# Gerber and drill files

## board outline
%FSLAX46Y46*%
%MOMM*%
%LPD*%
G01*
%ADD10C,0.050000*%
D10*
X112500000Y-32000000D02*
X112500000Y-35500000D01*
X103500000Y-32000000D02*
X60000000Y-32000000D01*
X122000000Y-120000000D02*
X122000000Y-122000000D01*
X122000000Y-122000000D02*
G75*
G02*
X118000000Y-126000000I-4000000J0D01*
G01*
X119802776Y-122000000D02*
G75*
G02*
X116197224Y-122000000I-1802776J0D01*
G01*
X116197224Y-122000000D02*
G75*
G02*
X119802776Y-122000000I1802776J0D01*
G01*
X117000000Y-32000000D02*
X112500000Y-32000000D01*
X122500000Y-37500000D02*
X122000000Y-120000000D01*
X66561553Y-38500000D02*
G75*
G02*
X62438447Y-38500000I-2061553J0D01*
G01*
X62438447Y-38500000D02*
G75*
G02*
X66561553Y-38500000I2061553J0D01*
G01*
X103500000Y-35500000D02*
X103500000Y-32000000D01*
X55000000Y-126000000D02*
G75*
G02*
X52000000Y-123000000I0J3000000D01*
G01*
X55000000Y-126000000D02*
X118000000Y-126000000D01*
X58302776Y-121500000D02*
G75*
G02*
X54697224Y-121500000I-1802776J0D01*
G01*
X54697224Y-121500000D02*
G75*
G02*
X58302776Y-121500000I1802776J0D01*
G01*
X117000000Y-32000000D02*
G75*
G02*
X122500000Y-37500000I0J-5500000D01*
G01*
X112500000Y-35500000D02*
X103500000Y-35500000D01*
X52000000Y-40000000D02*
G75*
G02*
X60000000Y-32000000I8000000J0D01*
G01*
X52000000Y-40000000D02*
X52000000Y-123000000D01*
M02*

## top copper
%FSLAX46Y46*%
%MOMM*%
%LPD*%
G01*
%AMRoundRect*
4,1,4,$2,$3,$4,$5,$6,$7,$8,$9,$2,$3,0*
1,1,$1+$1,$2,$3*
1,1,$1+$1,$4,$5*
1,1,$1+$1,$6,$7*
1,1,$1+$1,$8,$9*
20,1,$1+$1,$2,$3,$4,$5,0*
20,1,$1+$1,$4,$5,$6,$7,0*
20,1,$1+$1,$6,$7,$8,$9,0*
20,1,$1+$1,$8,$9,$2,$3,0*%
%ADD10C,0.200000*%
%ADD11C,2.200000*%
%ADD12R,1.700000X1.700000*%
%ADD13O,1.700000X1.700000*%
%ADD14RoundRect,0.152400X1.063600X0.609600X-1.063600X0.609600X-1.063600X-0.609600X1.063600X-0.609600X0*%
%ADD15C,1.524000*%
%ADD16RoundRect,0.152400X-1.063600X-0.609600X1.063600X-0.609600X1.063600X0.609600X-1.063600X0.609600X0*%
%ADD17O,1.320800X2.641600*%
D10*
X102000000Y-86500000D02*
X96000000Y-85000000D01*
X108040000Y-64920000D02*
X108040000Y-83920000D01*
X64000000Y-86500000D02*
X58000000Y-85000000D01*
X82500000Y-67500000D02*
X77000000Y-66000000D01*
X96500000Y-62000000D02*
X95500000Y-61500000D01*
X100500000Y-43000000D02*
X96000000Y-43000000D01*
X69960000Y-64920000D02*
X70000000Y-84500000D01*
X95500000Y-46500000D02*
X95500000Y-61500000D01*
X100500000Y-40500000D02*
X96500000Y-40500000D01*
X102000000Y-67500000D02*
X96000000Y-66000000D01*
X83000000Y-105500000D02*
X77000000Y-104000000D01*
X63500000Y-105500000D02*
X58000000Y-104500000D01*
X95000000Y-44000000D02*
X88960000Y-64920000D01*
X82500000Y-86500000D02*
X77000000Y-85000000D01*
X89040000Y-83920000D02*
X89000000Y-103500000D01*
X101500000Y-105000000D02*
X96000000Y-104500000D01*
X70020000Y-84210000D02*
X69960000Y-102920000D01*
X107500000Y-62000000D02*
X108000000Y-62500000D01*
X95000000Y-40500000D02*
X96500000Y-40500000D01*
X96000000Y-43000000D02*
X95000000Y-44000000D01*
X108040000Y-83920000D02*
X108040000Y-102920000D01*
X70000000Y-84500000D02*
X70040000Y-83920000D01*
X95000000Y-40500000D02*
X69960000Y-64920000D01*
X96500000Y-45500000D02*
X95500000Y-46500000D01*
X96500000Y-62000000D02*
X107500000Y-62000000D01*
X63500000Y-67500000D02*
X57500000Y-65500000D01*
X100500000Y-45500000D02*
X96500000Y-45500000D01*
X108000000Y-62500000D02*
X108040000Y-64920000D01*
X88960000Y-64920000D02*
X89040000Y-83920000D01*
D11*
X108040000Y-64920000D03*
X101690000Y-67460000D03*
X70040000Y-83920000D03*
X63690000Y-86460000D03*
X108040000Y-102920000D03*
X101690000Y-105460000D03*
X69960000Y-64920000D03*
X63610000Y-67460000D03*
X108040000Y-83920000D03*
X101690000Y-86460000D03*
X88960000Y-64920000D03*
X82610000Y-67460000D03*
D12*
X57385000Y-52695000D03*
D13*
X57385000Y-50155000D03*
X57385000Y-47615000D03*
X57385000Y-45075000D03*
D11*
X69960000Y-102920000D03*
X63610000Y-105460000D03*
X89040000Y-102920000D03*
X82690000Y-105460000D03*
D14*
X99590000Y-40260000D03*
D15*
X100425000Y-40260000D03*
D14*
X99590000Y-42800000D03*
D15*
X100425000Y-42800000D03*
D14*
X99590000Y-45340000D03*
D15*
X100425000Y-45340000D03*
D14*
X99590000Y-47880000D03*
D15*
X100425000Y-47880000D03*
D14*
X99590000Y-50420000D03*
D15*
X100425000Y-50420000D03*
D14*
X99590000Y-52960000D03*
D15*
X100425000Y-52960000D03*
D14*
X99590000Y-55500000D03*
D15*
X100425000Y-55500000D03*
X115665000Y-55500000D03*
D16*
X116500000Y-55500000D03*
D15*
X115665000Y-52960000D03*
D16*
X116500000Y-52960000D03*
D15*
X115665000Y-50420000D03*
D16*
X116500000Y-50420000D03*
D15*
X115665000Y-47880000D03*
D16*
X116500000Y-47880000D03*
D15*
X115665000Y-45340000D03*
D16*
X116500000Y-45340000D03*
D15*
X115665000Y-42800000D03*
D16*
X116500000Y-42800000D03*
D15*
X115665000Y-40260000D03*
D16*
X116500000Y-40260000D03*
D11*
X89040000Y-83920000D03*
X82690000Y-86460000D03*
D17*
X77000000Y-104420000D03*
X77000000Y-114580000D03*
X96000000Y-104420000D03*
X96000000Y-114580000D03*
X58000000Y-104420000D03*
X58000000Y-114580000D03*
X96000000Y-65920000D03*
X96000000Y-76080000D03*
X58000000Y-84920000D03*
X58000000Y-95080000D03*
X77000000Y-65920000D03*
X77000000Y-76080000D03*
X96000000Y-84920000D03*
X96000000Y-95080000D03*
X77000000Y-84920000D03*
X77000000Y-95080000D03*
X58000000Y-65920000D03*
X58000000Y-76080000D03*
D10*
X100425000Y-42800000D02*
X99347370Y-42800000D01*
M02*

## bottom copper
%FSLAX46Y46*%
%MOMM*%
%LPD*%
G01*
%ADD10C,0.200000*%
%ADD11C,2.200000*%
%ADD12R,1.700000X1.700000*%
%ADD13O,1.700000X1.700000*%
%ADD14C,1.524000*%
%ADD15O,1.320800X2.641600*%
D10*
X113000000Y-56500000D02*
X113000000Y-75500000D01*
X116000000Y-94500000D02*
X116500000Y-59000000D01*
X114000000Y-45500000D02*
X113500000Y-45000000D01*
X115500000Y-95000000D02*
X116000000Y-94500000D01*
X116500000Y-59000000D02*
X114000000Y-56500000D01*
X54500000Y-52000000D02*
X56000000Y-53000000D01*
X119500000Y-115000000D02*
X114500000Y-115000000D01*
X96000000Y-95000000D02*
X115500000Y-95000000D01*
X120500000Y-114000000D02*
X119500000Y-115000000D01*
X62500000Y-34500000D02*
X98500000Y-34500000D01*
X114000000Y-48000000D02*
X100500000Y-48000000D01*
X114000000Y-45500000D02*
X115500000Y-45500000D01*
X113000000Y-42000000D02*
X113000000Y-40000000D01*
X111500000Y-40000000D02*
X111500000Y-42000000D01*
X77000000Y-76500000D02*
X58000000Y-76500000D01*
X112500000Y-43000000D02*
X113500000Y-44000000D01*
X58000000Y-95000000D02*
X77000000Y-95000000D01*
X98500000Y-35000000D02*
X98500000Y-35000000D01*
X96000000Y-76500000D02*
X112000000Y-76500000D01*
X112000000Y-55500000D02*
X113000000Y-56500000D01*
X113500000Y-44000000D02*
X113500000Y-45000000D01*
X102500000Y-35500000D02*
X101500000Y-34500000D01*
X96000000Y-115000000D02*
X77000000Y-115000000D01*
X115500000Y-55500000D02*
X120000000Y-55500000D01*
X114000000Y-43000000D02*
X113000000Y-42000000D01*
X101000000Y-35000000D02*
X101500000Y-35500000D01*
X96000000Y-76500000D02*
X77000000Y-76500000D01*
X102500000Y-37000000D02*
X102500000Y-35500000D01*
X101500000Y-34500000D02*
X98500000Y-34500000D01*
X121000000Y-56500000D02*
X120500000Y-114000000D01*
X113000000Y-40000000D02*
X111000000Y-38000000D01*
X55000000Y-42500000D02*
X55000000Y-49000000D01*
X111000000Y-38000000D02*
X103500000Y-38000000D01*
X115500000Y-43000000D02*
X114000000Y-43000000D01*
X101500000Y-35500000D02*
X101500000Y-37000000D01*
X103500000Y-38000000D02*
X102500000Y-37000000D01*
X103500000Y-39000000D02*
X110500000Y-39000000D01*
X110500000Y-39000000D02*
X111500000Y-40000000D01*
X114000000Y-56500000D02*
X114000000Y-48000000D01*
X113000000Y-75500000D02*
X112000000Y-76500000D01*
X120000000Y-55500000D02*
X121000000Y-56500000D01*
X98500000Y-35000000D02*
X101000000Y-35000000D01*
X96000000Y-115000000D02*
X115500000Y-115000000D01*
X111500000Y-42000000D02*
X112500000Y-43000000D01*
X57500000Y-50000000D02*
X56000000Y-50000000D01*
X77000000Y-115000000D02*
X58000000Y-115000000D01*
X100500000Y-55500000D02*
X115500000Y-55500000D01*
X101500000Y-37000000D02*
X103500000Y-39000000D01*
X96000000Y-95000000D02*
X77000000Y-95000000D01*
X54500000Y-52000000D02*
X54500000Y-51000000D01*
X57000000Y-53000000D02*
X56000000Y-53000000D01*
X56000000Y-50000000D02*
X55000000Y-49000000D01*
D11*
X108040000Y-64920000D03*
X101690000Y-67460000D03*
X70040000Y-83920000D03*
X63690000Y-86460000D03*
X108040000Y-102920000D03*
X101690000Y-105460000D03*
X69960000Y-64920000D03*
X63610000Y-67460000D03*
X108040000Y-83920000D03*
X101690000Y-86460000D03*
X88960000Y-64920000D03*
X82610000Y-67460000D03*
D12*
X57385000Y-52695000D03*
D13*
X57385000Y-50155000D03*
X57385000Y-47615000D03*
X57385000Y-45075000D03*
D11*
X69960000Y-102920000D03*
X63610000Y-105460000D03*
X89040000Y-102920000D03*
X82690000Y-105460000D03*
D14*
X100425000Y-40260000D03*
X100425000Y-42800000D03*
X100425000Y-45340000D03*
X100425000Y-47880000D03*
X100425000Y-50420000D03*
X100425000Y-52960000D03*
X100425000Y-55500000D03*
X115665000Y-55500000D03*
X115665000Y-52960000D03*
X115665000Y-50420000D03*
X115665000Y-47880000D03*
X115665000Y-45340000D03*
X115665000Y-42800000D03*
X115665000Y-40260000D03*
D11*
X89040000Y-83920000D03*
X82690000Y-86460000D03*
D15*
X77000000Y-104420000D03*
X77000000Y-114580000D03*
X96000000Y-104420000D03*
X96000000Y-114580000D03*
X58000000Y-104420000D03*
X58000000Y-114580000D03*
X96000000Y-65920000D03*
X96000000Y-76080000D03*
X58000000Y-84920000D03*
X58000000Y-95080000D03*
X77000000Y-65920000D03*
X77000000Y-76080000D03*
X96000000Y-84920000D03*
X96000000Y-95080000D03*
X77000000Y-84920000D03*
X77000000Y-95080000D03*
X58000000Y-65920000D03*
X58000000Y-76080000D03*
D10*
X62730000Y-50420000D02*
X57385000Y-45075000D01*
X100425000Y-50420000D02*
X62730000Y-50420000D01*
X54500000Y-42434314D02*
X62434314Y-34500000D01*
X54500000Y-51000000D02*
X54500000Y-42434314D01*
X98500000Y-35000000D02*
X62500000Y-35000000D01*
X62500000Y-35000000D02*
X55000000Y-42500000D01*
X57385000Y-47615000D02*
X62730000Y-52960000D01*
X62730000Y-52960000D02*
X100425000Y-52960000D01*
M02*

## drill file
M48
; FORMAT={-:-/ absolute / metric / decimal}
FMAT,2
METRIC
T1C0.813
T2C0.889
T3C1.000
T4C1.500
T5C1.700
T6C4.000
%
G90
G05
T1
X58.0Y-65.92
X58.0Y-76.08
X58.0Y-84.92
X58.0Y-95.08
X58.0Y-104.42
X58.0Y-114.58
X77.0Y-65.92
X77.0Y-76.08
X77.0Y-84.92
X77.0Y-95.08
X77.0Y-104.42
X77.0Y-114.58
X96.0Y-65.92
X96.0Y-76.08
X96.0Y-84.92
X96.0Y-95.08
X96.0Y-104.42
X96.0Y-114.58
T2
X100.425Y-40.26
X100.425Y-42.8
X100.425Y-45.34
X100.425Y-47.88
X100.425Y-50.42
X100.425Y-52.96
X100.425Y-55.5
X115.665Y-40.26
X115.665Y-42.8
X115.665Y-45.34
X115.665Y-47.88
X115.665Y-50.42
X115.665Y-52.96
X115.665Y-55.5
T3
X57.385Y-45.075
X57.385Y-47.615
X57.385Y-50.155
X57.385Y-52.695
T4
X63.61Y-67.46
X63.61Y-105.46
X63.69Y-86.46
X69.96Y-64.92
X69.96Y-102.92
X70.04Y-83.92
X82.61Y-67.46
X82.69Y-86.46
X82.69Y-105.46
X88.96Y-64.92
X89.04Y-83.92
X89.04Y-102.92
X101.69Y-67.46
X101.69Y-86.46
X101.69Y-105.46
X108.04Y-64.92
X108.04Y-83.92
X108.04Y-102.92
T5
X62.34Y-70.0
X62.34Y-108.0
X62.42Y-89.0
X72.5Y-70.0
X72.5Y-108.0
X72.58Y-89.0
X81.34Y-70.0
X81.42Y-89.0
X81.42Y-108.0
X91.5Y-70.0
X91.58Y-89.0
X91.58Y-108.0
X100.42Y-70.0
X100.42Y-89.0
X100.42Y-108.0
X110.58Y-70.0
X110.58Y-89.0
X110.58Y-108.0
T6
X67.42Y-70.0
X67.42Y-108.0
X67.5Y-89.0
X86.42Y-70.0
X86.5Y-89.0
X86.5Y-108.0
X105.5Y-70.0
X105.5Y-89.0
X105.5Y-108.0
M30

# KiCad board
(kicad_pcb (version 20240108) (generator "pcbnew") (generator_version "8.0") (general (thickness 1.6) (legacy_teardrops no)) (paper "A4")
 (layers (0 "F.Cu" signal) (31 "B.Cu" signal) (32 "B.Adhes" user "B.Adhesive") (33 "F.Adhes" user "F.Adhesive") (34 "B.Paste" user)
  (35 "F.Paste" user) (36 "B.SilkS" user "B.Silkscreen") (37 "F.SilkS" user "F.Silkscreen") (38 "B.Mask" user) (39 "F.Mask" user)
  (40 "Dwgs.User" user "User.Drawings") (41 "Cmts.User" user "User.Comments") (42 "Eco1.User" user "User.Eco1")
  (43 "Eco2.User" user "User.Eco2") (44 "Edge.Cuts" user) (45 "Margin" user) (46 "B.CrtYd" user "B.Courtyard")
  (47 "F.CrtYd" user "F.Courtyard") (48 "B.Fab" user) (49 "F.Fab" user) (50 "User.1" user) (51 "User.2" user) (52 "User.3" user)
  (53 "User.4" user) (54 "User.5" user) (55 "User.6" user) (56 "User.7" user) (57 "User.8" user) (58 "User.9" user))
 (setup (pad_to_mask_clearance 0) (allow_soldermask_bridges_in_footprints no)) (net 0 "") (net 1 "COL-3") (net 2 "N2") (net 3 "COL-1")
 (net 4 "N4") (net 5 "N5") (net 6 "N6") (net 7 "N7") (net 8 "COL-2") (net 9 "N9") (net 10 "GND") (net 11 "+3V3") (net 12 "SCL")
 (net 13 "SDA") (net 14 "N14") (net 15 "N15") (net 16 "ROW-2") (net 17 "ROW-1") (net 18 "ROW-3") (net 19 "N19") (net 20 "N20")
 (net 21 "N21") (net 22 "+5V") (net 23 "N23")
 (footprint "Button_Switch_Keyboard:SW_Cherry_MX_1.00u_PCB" (layer "F.Cu") (at 108.04 64.92)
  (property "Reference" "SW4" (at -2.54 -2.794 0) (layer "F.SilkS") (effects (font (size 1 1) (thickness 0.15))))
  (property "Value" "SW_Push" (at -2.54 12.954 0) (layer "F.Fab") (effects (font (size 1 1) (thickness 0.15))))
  (pad "" np_thru_hole circle (at -7.62 5.08) (size 1.7 1.7) (drill 1.7) (layers "*.Cu" "*.Mask"))
  (pad "" np_thru_hole circle (at -2.54 5.08) (size 4 4) (drill 4) (layers "*.Cu" "*.Mask"))
  (pad "" np_thru_hole circle (at 2.54 5.08) (size 1.7 1.7) (drill 1.7) (layers "*.Cu" "*.Mask"))
  (pad "1" thru_hole circle (at 0 0) (size 2.2 2.2) (drill 1.5) (layers "*.Cu" "*.Mask") (remove_unused_layers no) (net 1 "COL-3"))
  (pad "2" thru_hole circle (at -6.35 2.54) (size 2.2 2.2) (drill 1.5) (layers "*.Cu" "*.Mask") (remove_unused_layers no) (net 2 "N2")))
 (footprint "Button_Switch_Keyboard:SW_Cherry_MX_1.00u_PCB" (layer "F.Cu") (at 70.04 83.92)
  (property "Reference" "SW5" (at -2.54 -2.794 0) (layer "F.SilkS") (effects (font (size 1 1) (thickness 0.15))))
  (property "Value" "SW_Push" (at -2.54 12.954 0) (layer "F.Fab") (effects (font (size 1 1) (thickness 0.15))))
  (pad "" np_thru_hole circle (at -7.62 5.08) (size 1.7 1.7) (drill 1.7) (layers "*.Cu" "*.Mask"))
  (pad "" np_thru_hole circle (at -2.54 5.08) (size 4 4) (drill 4) (layers "*.Cu" "*.Mask"))
  (pad "" np_thru_hole circle (at 2.54 5.08) (size 1.7 1.7) (drill 1.7) (layers "*.Cu" "*.Mask"))
  (pad "1" thru_hole circle (at 0 0) (size 2.2 2.2) (drill 1.5) (layers "*.Cu" "*.Mask") (remove_unused_layers no) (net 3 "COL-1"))
  (pad "2" thru_hole circle (at -6.35 2.54) (size 2.2 2.2) (drill 1.5) (layers "*.Cu" "*.Mask") (remove_unused_layers no) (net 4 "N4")))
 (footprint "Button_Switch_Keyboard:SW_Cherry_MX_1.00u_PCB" (layer "F.Cu") (at 108.04 102.92)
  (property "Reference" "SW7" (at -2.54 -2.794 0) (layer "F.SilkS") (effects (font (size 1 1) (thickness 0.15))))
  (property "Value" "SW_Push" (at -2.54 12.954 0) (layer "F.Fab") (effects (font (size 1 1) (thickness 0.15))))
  (pad "" np_thru_hole circle (at -7.62 5.08) (size 1.7 1.7) (drill 1.7) (layers "*.Cu" "*.Mask"))
  (pad "" np_thru_hole circle (at -2.54 5.08) (size 4 4) (drill 4) (layers "*.Cu" "*.Mask"))
  (pad "" np_thru_hole circle (at 2.54 5.08) (size 1.7 1.7) (drill 1.7) (layers "*.Cu" "*.Mask"))
  (pad "1" thru_hole circle (at 0 0) (size 2.2 2.2) (drill 1.5) (layers "*.Cu" "*.Mask") (remove_unused_layers no) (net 1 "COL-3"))
  (pad "2" thru_hole circle (at -6.35 2.54) (size 2.2 2.2) (drill 1.5) (layers "*.Cu" "*.Mask") (remove_unused_layers no) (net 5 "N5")))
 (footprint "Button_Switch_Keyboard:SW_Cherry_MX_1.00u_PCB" (layer "F.Cu") (at 69.96 64.92)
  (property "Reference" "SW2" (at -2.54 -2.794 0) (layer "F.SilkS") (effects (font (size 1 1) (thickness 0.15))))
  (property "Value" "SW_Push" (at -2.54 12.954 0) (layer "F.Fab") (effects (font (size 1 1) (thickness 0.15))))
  (pad "" np_thru_hole circle (at -7.62 5.08) (size 1.7 1.7) (drill 1.7) (layers "*.Cu" "*.Mask"))
  (pad "" np_thru_hole circle (at -2.54 5.08) (size 4 4) (drill 4) (layers "*.Cu" "*.Mask"))
  (pad "" np_thru_hole circle (at 2.54 5.08) (size 1.7 1.7) (drill 1.7) (layers "*.Cu" "*.Mask"))
  (pad "1" thru_hole circle (at 0 0) (size 2.2 2.2) (drill 1.5) (layers "*.Cu" "*.Mask") (remove_unused_layers no) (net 3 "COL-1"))
  (pad "2" thru_hole circle (at -6.35 2.54) (size 2.2 2.2) (drill 1.5) (layers "*.Cu" "*.Mask") (remove_unused_layers no) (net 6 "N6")))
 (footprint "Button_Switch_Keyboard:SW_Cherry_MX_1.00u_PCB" (layer "F.Cu") (at 108.04 83.92)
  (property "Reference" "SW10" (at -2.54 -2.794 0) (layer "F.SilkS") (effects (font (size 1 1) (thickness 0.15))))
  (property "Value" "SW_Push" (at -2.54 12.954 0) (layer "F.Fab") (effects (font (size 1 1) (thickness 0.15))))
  (pad "" np_thru_hole circle (at -7.62 5.08) (size 1.7 1.7) (drill 1.7) (layers "*.Cu" "*.Mask"))
  (pad "" np_thru_hole circle (at -2.54 5.08) (size 4 4) (drill 4) (layers "*.Cu" "*.Mask"))
  (pad "" np_thru_hole circle (at 2.54 5.08) (size 1.7 1.7) (drill 1.7) (layers "*.Cu" "*.Mask"))
  (pad "1" thru_hole circle (at 0 0) (size 2.2 2.2) (drill 1.5) (layers "*.Cu" "*.Mask") (remove_unused_layers no) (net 1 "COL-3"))
  (pad "2" thru_hole circle (at -6.35 2.54) (size 2.2 2.2) (drill 1.5) (layers "*.Cu" "*.Mask") (remove_unused_layers no) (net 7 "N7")))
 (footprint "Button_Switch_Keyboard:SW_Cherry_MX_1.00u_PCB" (layer "F.Cu") (at 88.96 64.92)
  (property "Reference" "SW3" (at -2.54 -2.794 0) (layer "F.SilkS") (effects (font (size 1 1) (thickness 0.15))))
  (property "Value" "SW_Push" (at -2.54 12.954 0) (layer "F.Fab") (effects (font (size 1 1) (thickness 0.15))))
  (pad "" np_thru_hole circle (at -7.62 5.08) (size 1.7 1.7) (drill 1.7) (layers "*.Cu" "*.Mask"))
  (pad "" np_thru_hole circle (at -2.54 5.08) (size 4 4) (drill 4) (layers "*.Cu" "*.Mask"))
  (pad "" np_thru_hole circle (at 2.54 5.08) (size 1.7 1.7) (drill 1.7) (layers "*.Cu" "*.Mask"))
  (pad "1" thru_hole circle (at 0 0) (size 2.2 2.2) (drill 1.5) (layers "*.Cu" "*.Mask") (remove_unused_layers no) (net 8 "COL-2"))
  (pad "2" thru_hole circle (at -6.35 2.54) (size 2.2 2.2) (drill 1.5) (layers "*.Cu" "*.Mask") (remove_unused_layers no) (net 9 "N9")))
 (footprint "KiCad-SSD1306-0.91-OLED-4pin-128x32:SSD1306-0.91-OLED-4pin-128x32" (layer "F.Cu") (at 93.885 54.885 180)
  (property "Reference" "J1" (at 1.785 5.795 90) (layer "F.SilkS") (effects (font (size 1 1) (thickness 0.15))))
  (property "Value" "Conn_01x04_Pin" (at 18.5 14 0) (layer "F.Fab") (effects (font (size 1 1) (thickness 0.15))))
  (pad "1" thru_hole rect (at 36.5 2.19 180) (size 1.7 1.7) (drill 1) (layers "*.Cu" "*.Mask") (remove_unused_layers no) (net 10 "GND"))
  (pad "2" thru_hole oval (at 36.5 4.73 180) (size 1.7 1.7) (drill 1) (layers "*.Cu" "*.Mask") (remove_unused_layers no) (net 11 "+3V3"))
  (pad "3" thru_hole oval (at 36.5 7.27 180) (size 1.7 1.7) (drill 1) (layers "*.Cu" "*.Mask") (remove_unused_layers no) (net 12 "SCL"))
  (pad "4" thru_hole oval (at 36.5 9.81 180) (size 1.7 1.7) (drill 1) (layers "*.Cu" "*.Mask") (remove_unused_layers no) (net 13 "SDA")))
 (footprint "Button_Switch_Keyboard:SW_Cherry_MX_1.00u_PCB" (layer "F.Cu") (at 69.96 102.92)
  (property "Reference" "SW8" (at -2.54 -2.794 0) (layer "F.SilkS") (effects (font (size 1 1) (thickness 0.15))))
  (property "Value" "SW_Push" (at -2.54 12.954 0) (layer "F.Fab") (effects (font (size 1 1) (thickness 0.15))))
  (pad "" np_thru_hole circle (at -7.62 5.08) (size 1.7 1.7) (drill 1.7) (layers "*.Cu" "*.Mask"))
  (pad "" np_thru_hole circle (at -2.54 5.08) (size 4 4) (drill 4) (layers "*.Cu" "*.Mask"))
  (pad "" np_thru_hole circle (at 2.54 5.08) (size 1.7 1.7) (drill 1.7) (layers "*.Cu" "*.Mask"))
  (pad "1" thru_hole circle (at 0 0) (size 2.2 2.2) (drill 1.5) (layers "*.Cu" "*.Mask") (remove_unused_layers no) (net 3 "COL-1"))
  (pad "2" thru_hole circle (at -6.35 2.54) (size 2.2 2.2) (drill 1.5) (layers "*.Cu" "*.Mask") (remove_unused_layers no) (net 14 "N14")))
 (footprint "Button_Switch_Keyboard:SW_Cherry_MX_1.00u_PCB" (layer "F.Cu") (at 89.04 102.92)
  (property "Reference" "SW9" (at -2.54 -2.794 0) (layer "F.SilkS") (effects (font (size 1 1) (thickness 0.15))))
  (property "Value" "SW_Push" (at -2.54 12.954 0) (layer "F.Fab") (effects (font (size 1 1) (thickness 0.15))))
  (pad "" np_thru_hole circle (at -7.62 5.08) (size 1.7 1.7) (drill 1.7) (layers "*.Cu" "*.Mask"))
  (pad "" np_thru_hole circle (at -2.54 5.08) (size 4 4) (drill 4) (layers "*.Cu" "*.Mask"))
  (pad "" np_thru_hole circle (at 2.54 5.08) (size 1.7 1.7) (drill 1.7) (layers "*.Cu" "*.Mask"))
  (pad "1" thru_hole circle (at 0 0) (size 2.2 2.2) (drill 1.5) (layers "*.Cu" "*.Mask") (remove_unused_layers no) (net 8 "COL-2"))
  (pad "2" thru_hole circle (at -6.35 2.54) (size 2.2 2.2) (drill 1.5) (layers "*.Cu" "*.Mask") (remove_unused_layers no) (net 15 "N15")))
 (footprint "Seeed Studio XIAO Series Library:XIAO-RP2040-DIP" (layer "F.Cu") (at 108.045 47.88)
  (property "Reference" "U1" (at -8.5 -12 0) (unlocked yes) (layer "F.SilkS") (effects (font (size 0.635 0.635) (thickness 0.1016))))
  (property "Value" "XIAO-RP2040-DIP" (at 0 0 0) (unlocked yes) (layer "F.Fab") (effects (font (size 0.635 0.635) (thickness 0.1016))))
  (pad "1" smd roundrect (at -8.455 -7.62 180) (size 2.432 1.524) (layers "F.Cu" "F.Mask") (roundrect_rratio 0.1) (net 3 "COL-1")
   (thermal_bridge_angle 45))
  (pad "1" thru_hole circle (at -7.62 -7.62 180) (size 1.524 1.524) (drill 0.889) (layers "*.Cu" "*.Mask") (remove_unused_layers no)
   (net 3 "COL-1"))
  (pad "2" smd roundrect (at -8.455 -5.08 180) (size 2.432 1.524) (layers "F.Cu" "F.Mask") (roundrect_rratio 0.1) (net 8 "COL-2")
   (thermal_bridge_angle 45))
  (pad "2" thru_hole circle (at -7.62 -5.08 180) (size 1.524 1.524) (drill 0.889) (layers "*.Cu" "*.Mask") (remove_unused_layers no)
   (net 8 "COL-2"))
  (pad "3" smd roundrect (at -8.455 -2.54 180) (size 2.432 1.524) (layers "F.Cu" "F.Mask") (roundrect_rratio 0.1) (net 1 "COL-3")
   (thermal_bridge_angle 45))
  (pad "3" thru_hole circle (at -7.62 -2.54 180) (size 1.524 1.524) (drill 0.889) (layers "*.Cu" "*.Mask") (remove_unused_layers no)
   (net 1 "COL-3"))
  (pad "4" smd roundrect (at -8.455 0 180) (size 2.432 1.524) (layers "F.Cu" "F.Mask") (roundrect_rratio 0.1) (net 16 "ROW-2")
   (thermal_bridge_angle 45))
  (pad "4" thru_hole circle (at -7.62 0 180) (size 1.524 1.524) (drill 0.889) (layers "*.Cu" "*.Mask") (remove_unused_layers no)
   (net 16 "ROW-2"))
  (pad "5" smd roundrect (at -8.455 2.54 180) (size 2.432 1.524) (layers "F.Cu" "F.Mask") (roundrect_rratio 0.1) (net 13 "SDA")
   (thermal_bridge_angle 45))
  (pad "5" thru_hole circle (at -7.62 2.54 180) (size 1.524 1.524) (drill 0.889) (layers "*.Cu" "*.Mask") (remove_unused_layers no)
   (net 13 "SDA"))
  (pad "6" smd roundrect (at -8.455 5.08 180) (size 2.432 1.524) (layers "F.Cu" "F.Mask") (roundrect_rratio 0.1) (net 12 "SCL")
   (thermal_bridge_angle 45))
  (pad "6" thru_hole circle (at -7.62 5.08 180) (size 1.524 1.524) (drill 0.889) (layers "*.Cu" "*.Mask") (remove_unused_layers no)
   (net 12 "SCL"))
  (pad "7" smd roundrect (at -8.455 7.62 180) (size 2.432 1.524) (layers "F.Cu" "F.Mask") (roundrect_rratio 0.1) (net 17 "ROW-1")
   (thermal_bridge_angle 45))
  (pad "7" thru_hole circle (at -7.62 7.62 180) (size 1.524 1.524) (drill 0.889) (layers "*.Cu" "*.Mask") (remove_unused_layers no)
   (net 17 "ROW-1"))
  (pad "8" thru_hole circle (at 7.62 7.62) (size 1.524 1.524) (drill 0.889) (layers "*.Cu" "*.Mask") (remove_unused_layers no)
   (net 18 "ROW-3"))
  (pad "8" smd roundrect (at 8.455 7.62) (size 2.432 1.524) (layers "F.Cu" "F.Mask") (roundrect_rratio 0.1) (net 18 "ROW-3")
   (thermal_bridge_angle 45))
  (pad "9" thru_hole circle (at 7.62 5.08) (size 1.524 1.524) (drill 0.889) (layers "*.Cu" "*.Mask") (remove_unused_layers no)
   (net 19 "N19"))
  (pad "9" smd roundrect (at 8.455 5.08) (size 2.432 1.524) (layers "F.Cu" "F.Mask") (roundrect_rratio 0.1) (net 19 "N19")
   (thermal_bridge_angle 45))
  (pad "10" thru_hole circle (at 7.62 2.54) (size 1.524 1.524) (drill 0.889) (layers "*.Cu" "*.Mask") (remove_unused_layers no)
   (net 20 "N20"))
  (pad "10" smd roundrect (at 8.455 2.54) (size 2.432 1.524) (layers "F.Cu" "F.Mask") (roundrect_rratio 0.1) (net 20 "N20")
   (thermal_bridge_angle 45))
  (pad "11" thru_hole circle (at 7.62 0) (size 1.524 1.524) (drill 0.889) (layers "*.Cu" "*.Mask") (remove_unused_layers no) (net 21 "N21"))
  (pad "11" smd roundrect (at 8.455 0) (size 2.432 1.524) (layers "F.Cu" "F.Mask") (roundrect_rratio 0.1) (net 21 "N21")
   (thermal_bridge_angle 45))
  (pad "12" thru_hole circle (at 7.62 -2.54) (size 1.524 1.524) (drill 0.889) (layers "*.Cu" "*.Mask") (remove_unused_layers no)
   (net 11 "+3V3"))
  (pad "12" smd roundrect (at 8.455 -2.54) (size 2.432 1.524) (layers "F.Cu" "F.Mask") (roundrect_rratio 0.1) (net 11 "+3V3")
   (thermal_bridge_angle 45))
  (pad "13" thru_hole circle (at 7.62 -5.08) (size 1.524 1.524) (drill 0.889) (layers "*.Cu" "*.Mask") (remove_unused_layers no)
   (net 10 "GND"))
  (pad "13" smd roundrect (at 8.455 -5.08) (size 2.432 1.524) (layers "F.Cu" "F.Mask") (roundrect_rratio 0.1) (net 10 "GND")
   (thermal_bridge_angle 45))
  (pad "14" thru_hole circle (at 7.62 -7.62) (size 1.524 1.524) (drill 0.889) (layers "*.Cu" "*.Mask") (remove_unused_layers no)
   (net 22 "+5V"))
  (pad "14" smd roundrect (at 8.455 -7.62) (size 2.432 1.524) (layers "F.Cu" "F.Mask") (roundrect_rratio 0.1) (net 22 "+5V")
   (thermal_bridge_angle 45)))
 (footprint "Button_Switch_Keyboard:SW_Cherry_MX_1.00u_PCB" (layer "F.Cu") (at 89.04 83.92)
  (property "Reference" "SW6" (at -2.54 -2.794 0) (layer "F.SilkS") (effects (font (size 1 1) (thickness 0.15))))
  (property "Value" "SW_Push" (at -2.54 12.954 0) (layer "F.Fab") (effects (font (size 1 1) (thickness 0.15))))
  (pad "" np_thru_hole circle (at -7.62 5.08) (size 1.7 1.7) (drill 1.7) (layers "*.Cu" "*.Mask"))
  (pad "" np_thru_hole circle (at -2.54 5.08) (size 4 4) (drill 4) (layers "*.Cu" "*.Mask"))
  (pad "" np_thru_hole circle (at 2.54 5.08) (size 1.7 1.7) (drill 1.7) (layers "*.Cu" "*.Mask"))
  (pad "1" thru_hole circle (at 0 0) (size 2.2 2.2) (drill 1.5) (layers "*.Cu" "*.Mask") (remove_unused_layers no) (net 8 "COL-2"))
  (pad "2" thru_hole circle (at -6.35 2.54) (size 2.2 2.2) (drill 1.5) (layers "*.Cu" "*.Mask") (remove_unused_layers no) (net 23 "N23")))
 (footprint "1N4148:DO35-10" (layer "B.Cu") (at 77 109.5 90)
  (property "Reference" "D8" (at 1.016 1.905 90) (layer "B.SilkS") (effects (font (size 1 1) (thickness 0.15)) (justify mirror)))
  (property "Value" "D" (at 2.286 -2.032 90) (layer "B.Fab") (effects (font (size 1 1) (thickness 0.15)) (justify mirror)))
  (pad "A" thru_hole oval (at 5.08 0 90) (size 2.6416 1.3208) (drill 0.8128) (layers "*.Cu" "*.Mask") (remove_unused_layers no)
   (solder_mask_margin 0.102))
  (pad "C" thru_hole oval (at -5.08 0 90) (size 2.6416 1.3208) (drill 0.8128) (layers "*.Cu" "*.Mask") (remove_unused_layers no)
   (solder_mask_margin 0.102)))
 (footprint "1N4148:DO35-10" (layer "B.Cu") (at 96 109.5 90)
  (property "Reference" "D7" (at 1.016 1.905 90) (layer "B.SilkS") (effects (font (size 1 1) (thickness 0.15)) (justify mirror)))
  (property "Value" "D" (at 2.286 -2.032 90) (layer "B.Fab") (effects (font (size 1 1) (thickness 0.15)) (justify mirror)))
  (pad "A" thru_hole oval (at 5.08 0 90) (size 2.6416 1.3208) (drill 0.8128) (layers "*.Cu" "*.Mask") (remove_unused_layers no)
   (solder_mask_margin 0.102))
  (pad "C" thru_hole oval (at -5.08 0 90) (size 2.6416 1.3208) (drill 0.8128) (layers "*.Cu" "*.Mask") (remove_unused_layers no)
   (solder_mask_margin 0.102)))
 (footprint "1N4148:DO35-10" (layer "B.Cu") (at 58 109.5 90)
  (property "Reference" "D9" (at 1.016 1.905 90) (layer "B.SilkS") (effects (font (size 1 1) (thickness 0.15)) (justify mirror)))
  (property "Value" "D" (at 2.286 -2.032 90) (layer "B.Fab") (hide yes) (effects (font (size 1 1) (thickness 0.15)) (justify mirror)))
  (pad "A" thru_hole oval (at 5.08 0 90) (size 2.6416 1.3208) (drill 0.8128) (layers "*.Cu" "*.Mask") (remove_unused_layers no)
   (solder_mask_margin 0.102))
  (pad "C" thru_hole oval (at -5.08 0 90) (size 2.6416 1.3208) (drill 0.8128) (layers "*.Cu" "*.Mask") (remove_unused_layers no)
   (solder_mask_margin 0.102)))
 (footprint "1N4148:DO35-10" (layer "B.Cu") (at 96 71 90)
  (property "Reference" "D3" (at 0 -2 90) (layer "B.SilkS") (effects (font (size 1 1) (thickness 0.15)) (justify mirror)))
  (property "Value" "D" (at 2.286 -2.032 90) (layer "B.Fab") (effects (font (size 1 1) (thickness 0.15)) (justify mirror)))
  (pad "A" thru_hole oval (at 5.08 0 90) (size 2.6416 1.3208) (drill 0.8128) (layers "*.Cu" "*.Mask") (remove_unused_layers no)
   (solder_mask_margin 0.102))
  (pad "C" thru_hole oval (at -5.08 0 90) (size 2.6416 1.3208) (drill 0.8128) (layers "*.Cu" "*.Mask") (remove_unused_layers no)
   (solder_mask_margin 0.102)))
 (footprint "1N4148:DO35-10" (layer "B.Cu") (at 58 90 90)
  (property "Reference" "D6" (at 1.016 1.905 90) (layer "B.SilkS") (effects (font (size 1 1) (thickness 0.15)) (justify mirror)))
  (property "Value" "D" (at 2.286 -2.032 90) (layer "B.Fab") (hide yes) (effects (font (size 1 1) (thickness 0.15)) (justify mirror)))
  (pad "A" thru_hole oval (at 5.08 0 90) (size 2.6416 1.3208) (drill 0.8128) (layers "*.Cu" "*.Mask") (remove_unused_layers no)
   (solder_mask_margin 0.102))
  (pad "C" thru_hole oval (at -5.08 0 90) (size 2.6416 1.3208) (drill 0.8128) (layers "*.Cu" "*.Mask") (remove_unused_layers no)
   (solder_mask_margin 0.102)))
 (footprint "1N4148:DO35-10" (layer "B.Cu") (at 77 71 90)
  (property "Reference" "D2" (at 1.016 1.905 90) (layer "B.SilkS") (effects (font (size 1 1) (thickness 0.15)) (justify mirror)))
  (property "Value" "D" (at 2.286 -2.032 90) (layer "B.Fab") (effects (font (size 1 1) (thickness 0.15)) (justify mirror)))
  (pad "A" thru_hole oval (at 5.08 0 90) (size 2.6416 1.3208) (drill 0.8128) (layers "*.Cu" "*.Mask") (remove_unused_layers no)
   (solder_mask_margin 0.102))
  (pad "C" thru_hole oval (at -5.08 0 90) (size 2.6416 1.3208) (drill 0.8128) (layers "*.Cu" "*.Mask") (remove_unused_layers no)
   (solder_mask_margin 0.102)))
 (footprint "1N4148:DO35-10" (layer "B.Cu") (at 96 90 90)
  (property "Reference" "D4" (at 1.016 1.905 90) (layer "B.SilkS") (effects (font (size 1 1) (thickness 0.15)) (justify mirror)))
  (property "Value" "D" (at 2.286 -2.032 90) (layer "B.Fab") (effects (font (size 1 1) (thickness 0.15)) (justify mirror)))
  (pad "A" thru_hole oval (at 5.08 0 90) (size 2.6416 1.3208) (drill 0.8128) (layers "*.Cu" "*.Mask") (remove_unused_layers no)
   (solder_mask_margin 0.102))
  (pad "C" thru_hole oval (at -5.08 0 90) (size 2.6416 1.3208) (drill 0.8128) (layers "*.Cu" "*.Mask") (remove_unused_layers no)
   (solder_mask_margin 0.102)))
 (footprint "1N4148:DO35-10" (layer "B.Cu") (at 77 90 90)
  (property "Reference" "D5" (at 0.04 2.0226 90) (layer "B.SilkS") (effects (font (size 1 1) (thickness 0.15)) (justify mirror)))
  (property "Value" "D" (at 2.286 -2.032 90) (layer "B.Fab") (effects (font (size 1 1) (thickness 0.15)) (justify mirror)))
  (pad "A" thru_hole oval (at 5.08 0 90) (size 2.6416 1.3208) (drill 0.8128) (layers "*.Cu" "*.Mask") (remove_unused_layers no)
   (solder_mask_margin 0.102))
  (pad "C" thru_hole oval (at -5.08 0 90) (size 2.6416 1.3208) (drill 0.8128) (layers "*.Cu" "*.Mask") (remove_unused_layers no)
   (solder_mask_margin 0.102)))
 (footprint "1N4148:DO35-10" (layer "B.Cu") (at 58 71 90)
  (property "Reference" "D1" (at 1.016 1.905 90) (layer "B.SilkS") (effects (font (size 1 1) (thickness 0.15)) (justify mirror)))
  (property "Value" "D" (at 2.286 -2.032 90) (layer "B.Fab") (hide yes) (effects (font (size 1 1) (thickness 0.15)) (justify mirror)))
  (pad "A" thru_hole oval (at 5.08 0 90) (size 2.6416 1.3208) (drill 0.8128) (layers "*.Cu" "*.Mask") (remove_unused_layers no)
   (solder_mask_margin 0.102))
  (pad "C" thru_hole oval (at -5.08 0 90) (size 2.6416 1.3208) (drill 0.8128) (layers "*.Cu" "*.Mask") (remove_unused_layers no)
   (solder_mask_margin 0.102)))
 (gr_line (start 102 86.5) (end 96 85) (stroke (width 0.2) (type default)) (layer "F.Cu") (net 7))
 (gr_line (start 108.04 64.92) (end 108.04 83.92) (stroke (width 0.2) (type default)) (layer "F.Cu") (net 1))
 (gr_line (start 64 86.5) (end 58 85) (stroke (width 0.2) (type default)) (layer "F.Cu") (net 4))
 (gr_line (start 82.5 67.5) (end 77 66) (stroke (width 0.2) (type default)) (layer "F.Cu") (net 9))
 (gr_line (start 96.5 62) (end 95.5 61.5) (stroke (width 0.2) (type default)) (layer "F.Cu") (net 1))
 (gr_line (start 100.5 43) (end 96 43) (stroke (width 0.2) (type default)) (layer "F.Cu") (net 8))
 (gr_line (start 69.96 64.92) (end 70 84.5) (stroke (width 0.2) (type default)) (layer "F.Cu") (net 3))
 (gr_line (start 95.5 46.5) (end 95.5 61.5) (stroke (width 0.2) (type default)) (layer "F.Cu") (net 1))
 (gr_line (start 100.5 40.5) (end 96.5 40.5) (stroke (width 0.2) (type default)) (layer "F.Cu") (net 3))
 (gr_line (start 102 67.5) (end 96 66) (stroke (width 0.2) (type default)) (layer "F.Cu") (net 2))
 (gr_line (start 83 105.5) (end 77 104) (stroke (width 0.2) (type default)) (layer "F.Cu") (net 15))
 (gr_line (start 63.5 105.5) (end 58 104.5) (stroke (width 0.2) (type default)) (layer "F.Cu") (net 14))
 (gr_line (start 95 44) (end 88.96 64.92) (stroke (width 0.2) (type default)) (layer "F.Cu") (net 8))
 (gr_line (start 82.5 86.5) (end 77 85) (stroke (width 0.2) (type default)) (layer "F.Cu") (net 23))
 (gr_line (start 89.04 83.92) (end 89 103.5) (stroke (width 0.2) (type default)) (layer "F.Cu") (net 8))
 (gr_line (start 101.5 105) (end 96 104.5) (stroke (width 0.2) (type default)) (layer "F.Cu") (net 5))
 (gr_line (start 70.02 84.21) (end 69.96 102.92) (stroke (width 0.2) (type default)) (layer "F.Cu") (net 3))
 (gr_line (start 107.5 62) (end 108 62.5) (stroke (width 0.2) (type default)) (layer "F.Cu") (net 1))
 (gr_line (start 95 40.5) (end 96.5 40.5) (stroke (width 0.2) (type default)) (layer "F.Cu") (net 3))
 (gr_line (start 96 43) (end 95 44) (stroke (width 0.2) (type default)) (layer "F.Cu") (net 8))
 (gr_line (start 108.04 83.92) (end 108.04 102.92) (stroke (width 0.2) (type default)) (layer "F.Cu") (net 1))
 (gr_line (start 70 84.5) (end 70.04 83.92) (stroke (width 0.2) (type default)) (layer "F.Cu") (net 3))
 (gr_line (start 95 40.5) (end 69.96 64.92) (stroke (width 0.2) (type default)) (layer "F.Cu") (net 3))
 (gr_line (start 96.5 45.5) (end 95.5 46.5) (stroke (width 0.2) (type default)) (layer "F.Cu") (net 1))
 (gr_line (start 96.5 62) (end 107.5 62) (stroke (width 0.2) (type default)) (layer "F.Cu") (net 1))
 (gr_line (start 63.5 67.5) (end 57.5 65.5) (stroke (width 0.2) (type default)) (layer "F.Cu") (net 6))
 (gr_line (start 100.5 45.5) (end 96.5 45.5) (stroke (width 0.2) (type default)) (layer "F.Cu") (net 1))
 (gr_line (start 108 62.5) (end 108.04 64.92) (stroke (width 0.2) (type default)) (layer "F.Cu") (net 1))
 (gr_line (start 88.96 64.92) (end 89.04 83.92) (stroke (width 0.2) (type default)) (layer "F.Cu") (net 8))
 (gr_line (start 113 56.5) (end 113 75.5) (stroke (width 0.2) (type default)) (layer "B.Cu") (net 17))
 (gr_line (start 116 94.5) (end 116.5 59) (stroke (width 0.2) (type default)) (layer "B.Cu") (net 16))
 (gr_line (start 114 45.5) (end 113.5 45) (stroke (width 0.2) (type default)) (layer "B.Cu") (net 11))
 (gr_line (start 115.5 95) (end 116 94.5) (stroke (width 0.2) (type default)) (layer "B.Cu") (net 16))
 (gr_line (start 116.5 59) (end 114 56.5) (stroke (width 0.2) (type default)) (layer "B.Cu") (net 16))
 (gr_line (start 54.5 52) (end 56 53) (stroke (width 0.2) (type default)) (layer "B.Cu") (net 10))
 (gr_line (start 119.5 115) (end 114.5 115) (stroke (width 0.2) (type default)) (layer "B.Cu") (net 18))
 (gr_line (start 96 95) (end 115.5 95) (stroke (width 0.2) (type default)) (layer "B.Cu") (net 16))
 (gr_line (start 120.5 114) (end 119.5 115) (stroke (width 0.2) (type default)) (layer "B.Cu") (net 18))
 (gr_line (start 62.5 34.5) (end 98.5 34.5) (stroke (width 0.2) (type default)) (layer "B.Cu") (net 10))
 (gr_line (start 114 48) (end 100.5 48) (stroke (width 0.2) (type default)) (layer "B.Cu") (net 16))
 (gr_line (start 114 45.5) (end 115.5 45.5) (stroke (width 0.2) (type default)) (layer "B.Cu") (net 11))
 (gr_line (start 113 42) (end 113 40) (stroke (width 0.2) (type default)) (layer "B.Cu") (net 10))
 (gr_line (start 111.5 40) (end 111.5 42) (stroke (width 0.2) (type default)) (layer "B.Cu") (net 11))
 (gr_line (start 77 76.5) (end 58 76.5) (stroke (width 0.2) (type default)) (layer "B.Cu") (net 17))
 (gr_line (start 112.5 43) (end 113.5 44) (stroke (width 0.2) (type default)) (layer "B.Cu") (net 11))
 (gr_line (start 58 95) (end 77 95) (stroke (width 0.2) (type default)) (layer "B.Cu") (net 16))
 (gr_line (start 98.5 35) (end 98.5 35) (stroke (width 0.2) (type default)) (layer "B.Cu") (net 11))
 (gr_line (start 96 76.5) (end 112 76.5) (stroke (width 0.2) (type default)) (layer "B.Cu") (net 17))
 (gr_line (start 112 55.5) (end 113 56.5) (stroke (width 0.2) (type default)) (layer "B.Cu") (net 17))
 (gr_line (start 113.5 44) (end 113.5 45) (stroke (width 0.2) (type default)) (layer "B.Cu") (net 11))
 (gr_line (start 102.5 35.5) (end 101.5 34.5) (stroke (width 0.2) (type default)) (layer "B.Cu") (net 10))
 (gr_line (start 96 115) (end 77 115) (stroke (width 0.2) (type default)) (layer "B.Cu") (net 18))
 (gr_line (start 115.5 55.5) (end 120 55.5) (stroke (width 0.2) (type default)) (layer "B.Cu") (net 18))
 (gr_line (start 114 43) (end 113 42) (stroke (width 0.2) (type default)) (layer "B.Cu") (net 10))
 (gr_line (start 101 35) (end 101.5 35.5) (stroke (width 0.2) (type default)) (layer "B.Cu") (net 11))
 (gr_line (start 96 76.5) (end 77 76.5) (stroke (width 0.2) (type default)) (layer "B.Cu") (net 17))
 (gr_line (start 102.5 37) (end 102.5 35.5) (stroke (width 0.2) (type default)) (layer "B.Cu") (net 10))
 (gr_line (start 101.5 34.5) (end 98.5 34.5) (stroke (width 0.2) (type default)) (layer "B.Cu") (net 10))
 (gr_line (start 121 56.5) (end 120.5 114) (stroke (width 0.2) (type default)) (layer "B.Cu") (net 18))
 (gr_line (start 113 40) (end 111 38) (stroke (width 0.2) (type default)) (layer "B.Cu") (net 10))
 (gr_line (start 55 42.5) (end 55 49) (stroke (width 0.2) (type default)) (layer "B.Cu") (net 11))
 (gr_line (start 111 38) (end 103.5 38) (stroke (width 0.2) (type default)) (layer "B.Cu") (net 10))
 (gr_line (start 115.5 43) (end 114 43) (stroke (width 0.2) (type default)) (layer "B.Cu") (net 10))
 (gr_line (start 101.5 35.5) (end 101.5 37) (stroke (width 0.2) (type default)) (layer "B.Cu") (net 11))
 (gr_line (start 103.5 38) (end 102.5 37) (stroke (width 0.2) (type default)) (layer "B.Cu") (net 10))
 (gr_line (start 103.5 39) (end 110.5 39) (stroke (width 0.2) (type default)) (layer "B.Cu") (net 11))
 (gr_line (start 110.5 39) (end 111.5 40) (stroke (width 0.2) (type default)) (layer "B.Cu") (net 11))
 (gr_line (start 114 56.5) (end 114 48) (stroke (width 0.2) (type default)) (layer "B.Cu") (net 16))
 (gr_line (start 113 75.5) (end 112 76.5) (stroke (width 0.2) (type default)) (layer "B.Cu") (net 17))
 (gr_line (start 120 55.5) (end 121 56.5) (stroke (width 0.2) (type default)) (layer "B.Cu") (net 18))
 (gr_line (start 98.5 35) (end 101 35) (stroke (width 0.2) (type default)) (layer "B.Cu") (net 11))
 (gr_line (start 96 115) (end 115.5 115) (stroke (width 0.2) (type default)) (layer "B.Cu") (net 18))
 (gr_line (start 111.5 42) (end 112.5 43) (stroke (width 0.2) (type default)) (layer "B.Cu") (net 11))
 (gr_line (start 57.5 50) (end 56 50) (stroke (width 0.2) (type default)) (layer "B.Cu") (net 11))
 (gr_line (start 77 115) (end 58 115) (stroke (width 0.2) (type default)) (layer "B.Cu") (net 18))
 (gr_line (start 100.5 55.5) (end 115.5 55.5) (stroke (width 0.2) (type default)) (layer "B.Cu") (net 17))
 (gr_line (start 101.5 37) (end 103.5 39) (stroke (width 0.2) (type default)) (layer "B.Cu") (net 11))
 (gr_line (start 96 95) (end 77 95) (stroke (width 0.2) (type default)) (layer "B.Cu") (net 16))
 (gr_line (start 54.5 52) (end 54.5 51) (stroke (width 0.2) (type default)) (layer "B.Cu") (net 10))
 (gr_line (start 57 53) (end 56 53) (stroke (width 0.2) (type default)) (layer "B.Cu") (net 10))
 (gr_line (start 56 50) (end 55 49) (stroke (width 0.2) (type default)) (layer "B.Cu") (net 11))
 (gr_line (start 112.5 32) (end 112.5 35.5) (stroke (width 0.05) (type default)) (layer "Edge.Cuts"))
 (gr_line (start 103.5 32) (end 60 32) (stroke (width 0.05) (type default)) (layer "Edge.Cuts"))
 (gr_line (start 122 120) (end 122 122) (stroke (width 0.05) (type default)) (layer "Edge.Cuts"))
 (gr_arc (start 122 122) (mid 120.828427 124.828427) (end 118 126) (stroke (width 0.05) (type default)) (layer "Edge.Cuts"))
 (gr_circle (center 118 122) (end 119.5 121) (stroke (width 0.05) (type default)) (fill none) (layer "Edge.Cuts"))
 (gr_line (start 117 32) (end 112.5 32) (stroke (width 0.05) (type default)) (layer "Edge.Cuts"))
 (gr_line (start 122.5 37.5) (end 122 120) (stroke (width 0.05) (type default)) (layer "Edge.Cuts"))
 (gr_circle (center 64.5 38.5) (end 66.5 38) (stroke (width 0.05) (type default)) (fill none) (layer "Edge.Cuts"))
 (gr_line (start 103.5 35.5) (end 103.5 32) (stroke (width 0.05) (type default)) (layer "Edge.Cuts"))
 (gr_arc (start 55 126) (mid 52.87868 125.12132) (end 52 123) (stroke (width 0.05) (type default)) (layer "Edge.Cuts"))
 (gr_line (start 55 126) (end 118 126) (stroke (width 0.05) (type default)) (layer "Edge.Cuts"))
 (gr_circle (center 56.5 121.5) (end 58 120.5) (stroke (width 0.05) (type default)) (fill none) (layer "Edge.Cuts"))
 (gr_arc (start 117 32) (mid 120.889087 33.610913) (end 122.5 37.5) (stroke (width 0.05) (type default)) (layer "Edge.Cuts"))
 (gr_line (start 112.5 35.5) (end 103.5 35.5) (stroke (width 0.05) (type default)) (layer "Edge.Cuts"))
 (gr_arc (start 52 40) (mid 54.343146 34.343146) (end 60 32) (stroke (width 0.05) (type default)) (layer "Edge.Cuts"))
 (gr_line (start 52 40) (end 52 123) (stroke (width 0.05) (type default)) (layer "Edge.Cuts"))
 (segment (start 62.73 50.42) (end 57.385 45.075) (width 0.2) (layer "B.Cu") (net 13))
 (segment (start 100.425 50.42) (end 62.73 50.42) (width 0.2) (layer "B.Cu") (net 13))
 (segment (start 54.5 42.434314) (end 62.434314 34.5) (width 0.2) (layer "B.Cu") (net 10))
 (segment (start 54.5 51) (end 54.5 42.434314) (width 0.2) (layer "B.Cu") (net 10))
 (segment (start 98.5 35) (end 62.5 35) (width 0.2) (layer "B.Cu") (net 11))
 (segment (start 62.5 35) (end 55 42.5) (width 0.2) (layer "B.Cu") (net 11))
 (segment (start 57.385 47.615) (end 62.73 52.96) (width 0.2) (layer "B.Cu") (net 12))
 (segment (start 62.73 52.96) (end 100.425 52.96) (width 0.2) (layer "B.Cu") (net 12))
 (segment (start 100.425 42.8) (end 99.34737 42.8) (width 0.2) (layer "F.Cu") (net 8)))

